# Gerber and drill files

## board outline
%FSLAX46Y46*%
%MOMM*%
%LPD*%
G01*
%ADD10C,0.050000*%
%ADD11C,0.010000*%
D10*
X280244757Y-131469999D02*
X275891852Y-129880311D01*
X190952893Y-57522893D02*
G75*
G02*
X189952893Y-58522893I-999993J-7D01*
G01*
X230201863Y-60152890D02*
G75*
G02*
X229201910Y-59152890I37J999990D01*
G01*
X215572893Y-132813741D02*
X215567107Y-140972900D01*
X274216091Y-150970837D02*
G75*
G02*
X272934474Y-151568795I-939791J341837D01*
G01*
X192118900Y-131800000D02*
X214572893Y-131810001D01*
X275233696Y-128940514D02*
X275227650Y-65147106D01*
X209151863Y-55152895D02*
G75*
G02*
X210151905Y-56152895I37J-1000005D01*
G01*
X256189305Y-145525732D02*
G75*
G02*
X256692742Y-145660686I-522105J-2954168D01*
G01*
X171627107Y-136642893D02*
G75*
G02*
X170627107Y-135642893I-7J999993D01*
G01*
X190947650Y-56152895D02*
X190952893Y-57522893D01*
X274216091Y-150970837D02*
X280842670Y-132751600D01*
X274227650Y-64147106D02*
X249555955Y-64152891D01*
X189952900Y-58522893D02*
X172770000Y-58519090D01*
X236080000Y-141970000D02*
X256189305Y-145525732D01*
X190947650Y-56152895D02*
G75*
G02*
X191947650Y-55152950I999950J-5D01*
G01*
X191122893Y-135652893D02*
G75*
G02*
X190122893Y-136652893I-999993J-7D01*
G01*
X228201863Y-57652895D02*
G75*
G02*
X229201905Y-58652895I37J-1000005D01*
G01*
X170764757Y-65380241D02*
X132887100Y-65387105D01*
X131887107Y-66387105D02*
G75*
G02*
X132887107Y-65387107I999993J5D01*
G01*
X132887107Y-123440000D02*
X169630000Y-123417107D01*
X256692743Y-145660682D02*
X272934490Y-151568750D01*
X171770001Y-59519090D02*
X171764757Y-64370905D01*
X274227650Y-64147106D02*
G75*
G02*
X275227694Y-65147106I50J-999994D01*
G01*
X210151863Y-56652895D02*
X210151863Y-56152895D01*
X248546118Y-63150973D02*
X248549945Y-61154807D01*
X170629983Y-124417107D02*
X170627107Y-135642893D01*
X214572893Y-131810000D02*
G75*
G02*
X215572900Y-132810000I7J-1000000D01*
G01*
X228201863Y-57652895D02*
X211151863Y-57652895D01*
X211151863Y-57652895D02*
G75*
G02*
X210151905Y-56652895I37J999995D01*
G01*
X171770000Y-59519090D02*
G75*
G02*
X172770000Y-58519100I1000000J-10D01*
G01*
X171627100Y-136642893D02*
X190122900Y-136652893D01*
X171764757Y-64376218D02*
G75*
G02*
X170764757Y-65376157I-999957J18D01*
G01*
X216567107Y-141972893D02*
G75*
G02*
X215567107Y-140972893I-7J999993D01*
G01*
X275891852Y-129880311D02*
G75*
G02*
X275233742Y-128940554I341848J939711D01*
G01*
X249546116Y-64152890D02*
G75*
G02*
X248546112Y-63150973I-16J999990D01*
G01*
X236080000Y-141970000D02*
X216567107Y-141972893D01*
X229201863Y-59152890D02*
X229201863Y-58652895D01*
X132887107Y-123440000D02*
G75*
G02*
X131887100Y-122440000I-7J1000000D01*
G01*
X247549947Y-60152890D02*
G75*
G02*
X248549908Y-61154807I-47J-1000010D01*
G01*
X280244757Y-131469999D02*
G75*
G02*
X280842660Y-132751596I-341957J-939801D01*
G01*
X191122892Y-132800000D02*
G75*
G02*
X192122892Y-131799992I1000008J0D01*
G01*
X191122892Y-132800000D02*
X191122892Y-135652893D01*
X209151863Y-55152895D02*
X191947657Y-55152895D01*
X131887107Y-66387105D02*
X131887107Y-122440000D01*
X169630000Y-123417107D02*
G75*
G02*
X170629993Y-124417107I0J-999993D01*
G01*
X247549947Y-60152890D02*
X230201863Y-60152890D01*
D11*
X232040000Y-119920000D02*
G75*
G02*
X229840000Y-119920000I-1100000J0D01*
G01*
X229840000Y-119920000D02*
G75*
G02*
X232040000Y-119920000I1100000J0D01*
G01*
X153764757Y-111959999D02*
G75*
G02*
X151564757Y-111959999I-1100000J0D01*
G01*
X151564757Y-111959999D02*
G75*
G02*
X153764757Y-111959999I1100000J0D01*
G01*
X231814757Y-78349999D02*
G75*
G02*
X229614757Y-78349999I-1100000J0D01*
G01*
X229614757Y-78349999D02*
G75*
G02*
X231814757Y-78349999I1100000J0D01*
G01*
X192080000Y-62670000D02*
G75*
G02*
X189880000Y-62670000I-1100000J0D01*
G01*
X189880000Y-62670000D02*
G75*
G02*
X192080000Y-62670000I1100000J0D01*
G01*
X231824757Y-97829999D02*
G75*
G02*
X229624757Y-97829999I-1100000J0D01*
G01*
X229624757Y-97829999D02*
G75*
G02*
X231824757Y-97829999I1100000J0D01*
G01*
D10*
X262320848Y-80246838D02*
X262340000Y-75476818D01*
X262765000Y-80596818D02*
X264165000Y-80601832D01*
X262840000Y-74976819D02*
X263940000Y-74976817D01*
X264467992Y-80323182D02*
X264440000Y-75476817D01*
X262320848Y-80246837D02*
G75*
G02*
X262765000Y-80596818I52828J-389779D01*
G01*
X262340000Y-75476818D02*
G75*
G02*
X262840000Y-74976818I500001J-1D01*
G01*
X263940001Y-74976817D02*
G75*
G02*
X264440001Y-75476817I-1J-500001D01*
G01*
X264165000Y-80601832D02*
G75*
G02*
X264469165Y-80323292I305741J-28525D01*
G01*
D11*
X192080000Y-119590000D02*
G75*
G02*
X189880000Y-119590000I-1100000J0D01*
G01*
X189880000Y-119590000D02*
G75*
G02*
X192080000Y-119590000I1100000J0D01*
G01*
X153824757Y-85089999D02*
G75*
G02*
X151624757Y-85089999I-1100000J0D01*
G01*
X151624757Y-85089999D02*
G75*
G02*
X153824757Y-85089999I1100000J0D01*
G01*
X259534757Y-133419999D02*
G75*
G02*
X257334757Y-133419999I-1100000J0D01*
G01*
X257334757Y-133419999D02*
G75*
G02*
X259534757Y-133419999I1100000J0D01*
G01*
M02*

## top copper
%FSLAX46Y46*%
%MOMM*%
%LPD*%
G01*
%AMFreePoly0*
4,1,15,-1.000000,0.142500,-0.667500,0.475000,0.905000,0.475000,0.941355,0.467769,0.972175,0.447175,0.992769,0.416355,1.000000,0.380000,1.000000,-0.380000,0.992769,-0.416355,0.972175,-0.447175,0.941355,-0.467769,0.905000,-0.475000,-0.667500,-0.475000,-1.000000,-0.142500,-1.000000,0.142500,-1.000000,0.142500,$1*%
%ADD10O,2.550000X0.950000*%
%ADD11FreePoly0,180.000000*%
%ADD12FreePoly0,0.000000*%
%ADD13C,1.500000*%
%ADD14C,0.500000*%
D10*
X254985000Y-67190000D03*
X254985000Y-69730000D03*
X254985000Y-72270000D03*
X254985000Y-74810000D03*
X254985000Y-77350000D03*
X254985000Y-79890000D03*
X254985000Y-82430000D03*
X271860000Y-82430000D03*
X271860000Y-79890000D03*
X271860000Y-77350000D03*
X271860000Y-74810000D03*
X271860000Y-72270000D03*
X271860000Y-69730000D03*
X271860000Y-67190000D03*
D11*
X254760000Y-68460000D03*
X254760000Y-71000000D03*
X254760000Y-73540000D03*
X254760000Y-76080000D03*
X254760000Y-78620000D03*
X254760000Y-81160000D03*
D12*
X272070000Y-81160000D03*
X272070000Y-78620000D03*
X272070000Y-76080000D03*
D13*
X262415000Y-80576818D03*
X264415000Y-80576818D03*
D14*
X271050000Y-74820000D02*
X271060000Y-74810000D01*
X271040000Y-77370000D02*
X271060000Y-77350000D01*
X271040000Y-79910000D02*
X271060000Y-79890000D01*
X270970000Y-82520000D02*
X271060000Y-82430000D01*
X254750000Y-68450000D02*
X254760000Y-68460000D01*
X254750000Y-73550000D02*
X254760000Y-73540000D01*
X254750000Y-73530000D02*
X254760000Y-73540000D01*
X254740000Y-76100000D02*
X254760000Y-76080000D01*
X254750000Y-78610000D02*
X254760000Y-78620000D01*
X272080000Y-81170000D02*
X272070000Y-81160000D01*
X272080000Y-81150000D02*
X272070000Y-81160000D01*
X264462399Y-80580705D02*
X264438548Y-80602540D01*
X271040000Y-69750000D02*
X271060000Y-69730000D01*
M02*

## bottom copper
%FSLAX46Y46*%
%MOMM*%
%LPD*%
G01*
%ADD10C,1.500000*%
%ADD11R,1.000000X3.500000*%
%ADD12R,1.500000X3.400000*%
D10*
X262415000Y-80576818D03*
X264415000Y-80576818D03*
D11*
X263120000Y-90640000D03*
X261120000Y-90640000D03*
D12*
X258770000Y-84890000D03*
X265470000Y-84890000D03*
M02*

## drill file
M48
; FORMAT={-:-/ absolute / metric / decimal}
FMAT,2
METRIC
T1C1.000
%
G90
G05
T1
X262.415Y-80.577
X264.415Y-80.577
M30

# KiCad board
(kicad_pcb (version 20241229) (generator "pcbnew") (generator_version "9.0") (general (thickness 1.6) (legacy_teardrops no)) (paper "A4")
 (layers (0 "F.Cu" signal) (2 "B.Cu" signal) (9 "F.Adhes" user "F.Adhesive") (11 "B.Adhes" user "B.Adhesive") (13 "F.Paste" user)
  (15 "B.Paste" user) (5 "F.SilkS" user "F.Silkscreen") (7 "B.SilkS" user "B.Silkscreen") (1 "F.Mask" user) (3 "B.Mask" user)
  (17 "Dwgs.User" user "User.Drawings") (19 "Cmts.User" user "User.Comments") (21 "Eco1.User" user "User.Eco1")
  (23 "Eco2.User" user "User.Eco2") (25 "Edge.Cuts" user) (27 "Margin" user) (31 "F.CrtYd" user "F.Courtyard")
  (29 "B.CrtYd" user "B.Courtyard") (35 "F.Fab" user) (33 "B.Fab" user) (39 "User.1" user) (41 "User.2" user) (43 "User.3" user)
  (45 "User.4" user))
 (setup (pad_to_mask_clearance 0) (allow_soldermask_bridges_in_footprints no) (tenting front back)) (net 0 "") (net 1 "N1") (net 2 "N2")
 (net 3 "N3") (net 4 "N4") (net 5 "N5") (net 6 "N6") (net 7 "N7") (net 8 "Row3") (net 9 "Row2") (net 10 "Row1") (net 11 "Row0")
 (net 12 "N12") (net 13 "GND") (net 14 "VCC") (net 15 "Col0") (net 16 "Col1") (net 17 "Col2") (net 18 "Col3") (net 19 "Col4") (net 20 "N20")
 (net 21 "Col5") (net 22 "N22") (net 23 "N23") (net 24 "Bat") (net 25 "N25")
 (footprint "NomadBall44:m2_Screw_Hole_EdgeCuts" (layer "F.Cu") (at 230.94 119.92)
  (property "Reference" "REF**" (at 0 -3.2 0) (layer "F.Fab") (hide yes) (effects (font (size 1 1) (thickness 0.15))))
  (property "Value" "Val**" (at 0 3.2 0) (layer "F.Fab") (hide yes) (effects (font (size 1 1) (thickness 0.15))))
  (fp_circle (center 0 0) (end 1.1 0) (stroke (width 0.01) (type solid)) (fill no) (layer "Edge.Cuts")))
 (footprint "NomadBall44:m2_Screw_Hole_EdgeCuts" (layer "F.Cu") (at 152.664757 111.959999)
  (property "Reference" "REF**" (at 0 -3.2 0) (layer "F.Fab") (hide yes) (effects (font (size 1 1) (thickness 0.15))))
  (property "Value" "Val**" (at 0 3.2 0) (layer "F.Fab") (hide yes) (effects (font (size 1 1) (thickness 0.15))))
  (fp_circle (center 0 0) (end 1.1 0) (stroke (width 0.01) (type solid)) (fill no) (layer "Edge.Cuts")))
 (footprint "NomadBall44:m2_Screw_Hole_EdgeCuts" (layer "F.Cu") (at 230.714757 78.349999)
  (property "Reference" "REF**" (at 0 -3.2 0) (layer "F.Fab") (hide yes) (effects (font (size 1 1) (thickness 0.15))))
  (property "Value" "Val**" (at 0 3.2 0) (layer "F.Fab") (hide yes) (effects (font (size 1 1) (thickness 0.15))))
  (fp_circle (center 0 0) (end 1.1 0) (stroke (width 0.01) (type solid)) (fill no) (layer "Edge.Cuts")))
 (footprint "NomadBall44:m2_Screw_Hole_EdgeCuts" (layer "F.Cu") (at 190.98 62.67)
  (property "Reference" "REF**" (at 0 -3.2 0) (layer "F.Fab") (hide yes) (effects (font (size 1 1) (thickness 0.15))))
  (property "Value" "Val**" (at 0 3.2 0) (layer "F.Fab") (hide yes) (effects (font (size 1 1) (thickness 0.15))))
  (fp_circle (center 0 0) (end 1.1 0) (stroke (width 0.01) (type solid)) (fill no) (layer "Edge.Cuts")))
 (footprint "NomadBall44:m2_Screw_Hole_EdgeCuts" (layer "F.Cu") (at 230.724757 97.829999)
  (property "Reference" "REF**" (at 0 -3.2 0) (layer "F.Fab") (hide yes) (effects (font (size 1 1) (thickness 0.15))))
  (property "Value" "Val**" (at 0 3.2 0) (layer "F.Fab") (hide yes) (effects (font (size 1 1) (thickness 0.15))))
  (fp_circle (center 0 0) (end 1.1 0) (stroke (width 0.01) (type solid)) (fill no) (layer "Edge.Cuts")))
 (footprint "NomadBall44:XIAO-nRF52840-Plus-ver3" (layer "F.Cu") (at 262.015 74.71 90)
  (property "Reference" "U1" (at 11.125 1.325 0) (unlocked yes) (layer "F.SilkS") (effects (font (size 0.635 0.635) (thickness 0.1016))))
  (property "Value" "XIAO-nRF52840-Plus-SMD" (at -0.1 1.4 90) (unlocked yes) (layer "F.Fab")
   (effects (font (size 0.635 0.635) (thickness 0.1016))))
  (fp_line (start -5.536838 0.305848) (end -0.766818 0.325) (stroke (width 0.05) (type default)) (layer "Edge.Cuts"))
  (fp_line (start -5.886818 0.75) (end -5.891832 2.15) (stroke (width 0.05) (type default)) (layer "Edge.Cuts"))
  (fp_line (start -0.266819 0.825) (end -0.266817 1.925) (stroke (width 0.05) (type default)) (layer "Edge.Cuts"))
  (fp_line (start -5.613182 2.452992) (end -0.766817 2.425) (stroke (width 0.05) (type default)) (layer "Edge.Cuts"))
  (fp_arc (start -5.536837 0.305848) (mid -5.617663 0.602123) (end -5.886818 0.75) (stroke (width 0.05) (type default)) (layer "Edge.Cuts"))
  (fp_arc (start -0.766818 0.325) (mid -0.413265 0.471447) (end -0.266818 0.825) (stroke (width 0.05) (type default)) (layer "Edge.Cuts"))
  (fp_arc (start -0.266817 1.925001) (mid -0.413264 2.278554) (end -0.766817 2.425001) (stroke (width 0.05) (type default))
   (layer "Edge.Cuts"))
  (fp_arc (start -5.891832 2.15) (mid -5.693897 2.24836) (end -5.613293 2.454165) (stroke (width 0.05) (type default)) (layer "Edge.Cuts"))
  (pad "1" smd oval (at 7.52 -6.23) (size 2.55 0.95) (drill (offset -0.8 0)) (layers "F.Cu" "F.Mask" "F.Paste") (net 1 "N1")
   (thermal_bridge_angle 45))
  (pad "2" smd oval (at 4.98 -6.23) (size 2.55 0.95) (drill (offset -0.8 0)) (layers "F.Cu" "F.Mask" "F.Paste") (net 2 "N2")
   (thermal_bridge_angle 45))
  (pad "3" smd oval (at 2.44 -6.23) (size 2.55 0.95) (drill (offset -0.8 0)) (layers "F.Cu" "F.Mask" "F.Paste") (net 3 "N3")
   (thermal_bridge_angle 45))
  (pad "4" smd oval (at -0.1 -6.23) (size 2.55 0.95) (drill (offset -0.8 0)) (layers "F.Cu" "F.Mask" "F.Paste") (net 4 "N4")
   (thermal_bridge_angle 45))
  (pad "5" smd oval (at -2.64 -6.23) (size 2.55 0.95) (drill (offset -0.8 0)) (layers "F.Cu" "F.Mask" "F.Paste") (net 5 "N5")
   (thermal_bridge_angle 45))
  (pad "6" smd oval (at -5.18 -6.23) (size 2.55 0.95) (drill (offset -0.8 0)) (layers "F.Cu" "F.Mask" "F.Paste") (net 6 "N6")
   (thermal_bridge_angle 45))
  (pad "7" smd oval (at -7.72 -6.23) (size 2.55 0.95) (drill (offset -0.8 0)) (layers "F.Cu" "F.Mask" "F.Paste") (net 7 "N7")
   (thermal_bridge_angle 45))
  (pad "8" smd oval (at -7.72 9.045) (size 2.55 0.95) (drill (offset 0.8 0)) (layers "F.Cu" "F.Mask" "F.Paste") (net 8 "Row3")
   (thermal_bridge_angle 45))
  (pad "9" smd oval (at -5.18 9.045) (size 2.55 0.95) (drill (offset 0.8 0)) (layers "F.Cu" "F.Mask" "F.Paste") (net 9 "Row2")
   (thermal_bridge_angle 45))
  (pad "10" smd oval (at -2.64 9.045) (size 2.55 0.95) (drill (offset 0.8 0)) (layers "F.Cu" "F.Mask" "F.Paste") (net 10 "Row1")
   (thermal_bridge_angle 45))
  (pad "11" smd oval (at -0.1 9.045) (size 2.55 0.95) (drill (offset 0.8 0)) (layers "F.Cu" "F.Mask" "F.Paste") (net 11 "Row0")
   (thermal_bridge_angle 45))
  (pad "12" smd oval (at 2.44 9.045) (size 2.55 0.95) (drill (offset 0.8 0)) (layers "F.Cu" "F.Mask" "F.Paste") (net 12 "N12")
   (thermal_bridge_angle 45))
  (pad "13" smd oval (at 4.98 9.045) (size 2.55 0.95) (drill (offset 0.8 0)) (layers "F.Cu" "F.Mask" "F.Paste") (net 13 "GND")
   (thermal_bridge_angle 45))
  (pad "14" smd oval (at 7.52 9.045) (size 2.55 0.95) (drill (offset 0.8 0)) (layers "F.Cu" "F.Mask" "F.Paste") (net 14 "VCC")
   (thermal_bridge_angle 45))
  (pad "15" smd roundrect (at 6.25 -7.255 180) (size 2 0.95) (layers "F.Cu" "F.Mask" "F.Paste") (roundrect_rratio 0.1) (chamfer_ratio 0.35)
   (chamfer top_left bottom_left) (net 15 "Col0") (thermal_bridge_angle 45))
  (pad "16" smd roundrect (at 3.71 -7.255 180) (size 2 0.95) (layers "F.Cu" "F.Mask" "F.Paste") (roundrect_rratio 0.1) (chamfer_ratio 0.35)
   (chamfer top_left bottom_left) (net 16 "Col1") (thermal_bridge_angle 45))
  (pad "17" smd roundrect (at 1.17 -7.255 180) (size 2 0.95) (layers "F.Cu" "F.Mask" "F.Paste") (roundrect_rratio 0.1) (chamfer_ratio 0.35)
   (chamfer top_left bottom_left) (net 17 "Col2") (thermal_bridge_angle 45))
  (pad "18" smd roundrect (at -1.37 -7.255 180) (size 2 0.95) (layers "F.Cu" "F.Mask" "F.Paste") (roundrect_rratio 0.1) (chamfer_ratio 0.35)
   (chamfer top_left bottom_left) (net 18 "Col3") (thermal_bridge_angle 45))
  (pad "19" smd roundrect (at -3.91 -7.255 180) (size 2 0.95) (layers "F.Cu" "F.Mask" "F.Paste") (roundrect_rratio 0.1) (chamfer_ratio 0.35)
   (chamfer top_left bottom_left) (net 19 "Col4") (thermal_bridge_angle 45))
  (pad "20" smd roundrect (at -6.45 -7.255 180) (size 2 0.95) (layers "F.Cu" "F.Mask" "F.Paste") (roundrect_rratio 0.1) (chamfer_ratio 0.35)
   (chamfer top_left bottom_left) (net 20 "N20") (thermal_bridge_angle 45))
  (pad "21" smd roundrect (at -6.45 10.055) (size 2 0.95) (layers "F.Cu" "F.Mask" "F.Paste") (roundrect_rratio 0.1) (chamfer_ratio 0.35)
   (chamfer top_left bottom_left) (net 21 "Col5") (thermal_bridge_angle 45))
  (pad "22" smd roundrect (at -3.91 10.055) (size 2 0.95) (layers "F.Cu" "F.Mask" "F.Paste") (roundrect_rratio 0.1) (chamfer_ratio 0.35)
   (chamfer top_left bottom_left) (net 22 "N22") (thermal_bridge_angle 45))
  (pad "23" smd roundrect (at -1.37 10.055) (size 2 0.95) (layers "F.Cu" "F.Mask" "F.Paste") (roundrect_rratio 0.1) (chamfer_ratio 0.35)
   (chamfer top_left bottom_left) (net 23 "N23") (thermal_bridge_angle 45))
  (pad "32" thru_hole circle (at -5.866818 0.4 90) (size 1.5 1.5) (drill 1) (layers "*.Cu" "*.Mask") (remove_unused_layers no)
   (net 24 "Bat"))
  (pad "33" thru_hole circle (at -5.866818 2.4 90) (size 1.5 1.5) (drill 1) (layers "*.Cu" "*.Mask") (remove_unused_layers no)
   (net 13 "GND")))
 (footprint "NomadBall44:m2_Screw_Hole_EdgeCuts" (layer "F.Cu") (at 190.98 119.59)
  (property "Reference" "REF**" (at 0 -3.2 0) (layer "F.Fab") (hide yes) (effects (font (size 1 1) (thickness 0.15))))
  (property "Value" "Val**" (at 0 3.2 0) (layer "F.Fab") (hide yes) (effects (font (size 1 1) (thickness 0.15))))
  (fp_circle (center 0 0) (end 1.1 0) (stroke (width 0.01) (type solid)) (fill no) (layer "Edge.Cuts")))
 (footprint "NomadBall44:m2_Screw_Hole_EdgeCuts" (layer "F.Cu") (at 152.724757 85.089999)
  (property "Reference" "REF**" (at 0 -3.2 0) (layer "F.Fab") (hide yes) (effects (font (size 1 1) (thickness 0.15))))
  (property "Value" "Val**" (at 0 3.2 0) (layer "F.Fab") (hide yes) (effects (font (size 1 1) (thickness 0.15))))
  (fp_circle (center 0 0) (end 1.1 0) (stroke (width 0.01) (type solid)) (fill no) (layer "Edge.Cuts")))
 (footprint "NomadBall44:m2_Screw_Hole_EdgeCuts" (layer "F.Cu") (at 258.434757 133.419999)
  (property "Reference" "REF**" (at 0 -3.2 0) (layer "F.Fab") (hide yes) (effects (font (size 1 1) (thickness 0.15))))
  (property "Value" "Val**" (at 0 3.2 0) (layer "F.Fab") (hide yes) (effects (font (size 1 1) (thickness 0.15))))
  (fp_circle (center 0 0) (end 1.1 0) (stroke (width 0.01) (type solid)) (fill no) (layer "Edge.Cuts")))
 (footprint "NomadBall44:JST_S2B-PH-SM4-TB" (layer "B.Cu") (at 262.12 90.64 180)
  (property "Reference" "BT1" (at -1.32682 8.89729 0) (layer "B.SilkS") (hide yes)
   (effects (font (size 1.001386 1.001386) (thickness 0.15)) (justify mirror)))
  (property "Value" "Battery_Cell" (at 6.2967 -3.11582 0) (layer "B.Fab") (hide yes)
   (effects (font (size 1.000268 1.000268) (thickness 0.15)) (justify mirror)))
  (pad "1" smd rect (at -1 0 180) (size 1 3.5) (layers "B.Cu" "B.Mask" "B.Paste") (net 24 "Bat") (solder_mask_margin 0.102))
  (pad "2" smd rect (at 1 0 180) (size 1 3.5) (layers "B.Cu" "B.Mask" "B.Paste") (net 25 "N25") (solder_mask_margin 0.102))
  (pad "P1" smd rect (at 3.35 5.75 180) (size 1.5 3.4) (layers "B.Cu" "B.Mask" "B.Paste") (solder_mask_margin 0.102))
  (pad "P2" smd rect (at -3.35 5.75 180) (size 1.5 3.4) (layers "B.Cu" "B.Mask" "B.Paste") (solder_mask_margin 0.102)))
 (gr_line (start 280.244757 131.469999) (end 275.891852 129.880311) (stroke (width 0.05) (type solid)) (layer "Edge.Cuts"))
 (gr_arc (start 190.952893 57.522893) (mid 190.66 58.23) (end 189.952893 58.522893) (stroke (width 0.05) (type solid)) (layer "Edge.Cuts"))
 (gr_arc (start 230.201863 60.15289) (mid 229.494756 59.859997) (end 229.201863 59.15289) (stroke (width 0.05) (type solid))
  (layer "Edge.Cuts"))
 (gr_line (start 215.572893 132.813741) (end 215.567107 140.9729) (stroke (width 0.05) (type default)) (layer "Edge.Cuts"))
 (gr_arc (start 274.216091 150.970837) (mid 273.699122 151.535222) (end 272.93449 151.56875) (stroke (width 0.05) (type solid))
  (layer "Edge.Cuts"))
 (gr_line (start 192.1189 131.8) (end 214.572893 131.810001) (stroke (width 0.05) (type default)) (layer "Edge.Cuts"))
 (gr_line (start 275.233696 128.940514) (end 275.22765 65.147106) (stroke (width 0.05) (type solid)) (layer "Edge.Cuts"))
 (gr_arc (start 209.151863 55.152895) (mid 209.85897 55.445788) (end 210.151863 56.152895) (stroke (width 0.05) (type solid))
  (layer "Edge.Cuts"))
 (gr_arc (start 256.189305 145.525732) (mid 256.443961 145.582253) (end 256.692744 145.660682) (stroke (width 0.05) (type solid))
  (layer "Edge.Cuts"))
 (gr_arc (start 171.627107 136.642893) (mid 170.92 136.35) (end 170.627107 135.642893) (stroke (width 0.05) (type solid))
  (layer "Edge.Cuts"))
 (gr_line (start 190.94765 56.152895) (end 190.952893 57.522893) (stroke (width 0.05) (type solid)) (layer "Edge.Cuts"))
 (gr_line (start 274.216091 150.970837) (end 280.84267 132.7516) (stroke (width 0.05) (type solid)) (layer "Edge.Cuts"))
 (gr_line (start 274.22765 64.147106) (end 249.555955 64.152891) (stroke (width 0.05) (type solid)) (layer "Edge.Cuts"))
 (gr_line (start 189.9529 58.522893) (end 172.77 58.51909) (stroke (width 0.05) (type solid)) (layer "Edge.Cuts"))
 (gr_line (start 236.08 141.97) (end 256.189305 145.525732) (stroke (width 0.05) (type solid)) (layer "Edge.Cuts"))
 (gr_arc (start 190.94765 56.152895) (mid 191.240543 55.445788) (end 191.94765 55.152895) (stroke (width 0.05) (type solid))
  (layer "Edge.Cuts"))
 (gr_arc (start 191.122893 135.652893) (mid 190.83 136.36) (end 190.122893 136.652893) (stroke (width 0.05) (type solid))
  (layer "Edge.Cuts"))
 (gr_arc (start 228.201863 57.652895) (mid 228.90897 57.945788) (end 229.201863 58.652895) (stroke (width 0.05) (type solid))
  (layer "Edge.Cuts"))
 (gr_line (start 170.764757 65.380241) (end 132.8871 65.387105) (stroke (width 0.05) (type solid)) (layer "Edge.Cuts"))
 (gr_arc (start 131.887107 66.387105) (mid 132.18 65.679998) (end 132.887107 65.387105) (stroke (width 0.05) (type solid))
  (layer "Edge.Cuts"))
 (gr_line (start 132.887107 123.44) (end 169.63 123.417107) (stroke (width 0.05) (type solid)) (layer "Edge.Cuts"))
 (gr_line (start 256.692743 145.660682) (end 272.93449 151.56875) (stroke (width 0.05) (type solid)) (layer "Edge.Cuts"))
 (gr_line (start 171.770001 59.51909) (end 171.764757 64.370905) (stroke (width 0.05) (type solid)) (layer "Edge.Cuts"))
 (gr_arc (start 274.22765 64.147106) (mid 274.934757 64.439999) (end 275.22765 65.147106) (stroke (width 0.05) (type solid))
  (layer "Edge.Cuts"))
 (gr_line (start 210.151863 56.652895) (end 210.151863 56.152895) (stroke (width 0.05) (type solid)) (layer "Edge.Cuts"))
 (gr_line (start 248.546118 63.150973) (end 248.549945 61.154807) (stroke (width 0.05) (type solid)) (layer "Edge.Cuts"))
 (gr_line (start 170.629983 124.417107) (end 170.627107 135.642893) (stroke (width 0.05) (type default)) (layer "Edge.Cuts"))
 (gr_arc (start 214.572893 131.81) (mid 215.28 132.102893) (end 215.572893 132.81) (stroke (width 0.05) (type solid)) (layer "Edge.Cuts"))
 (gr_line (start 228.201863 57.652895) (end 211.151863 57.652895) (stroke (width 0.05) (type solid)) (layer "Edge.Cuts"))
 (gr_arc (start 211.151863 57.652895) (mid 210.444756 57.360002) (end 210.151863 56.652895) (stroke (width 0.05) (type solid))
  (layer "Edge.Cuts"))
 (gr_arc (start 171.77 59.51909) (mid 172.062893 58.811983) (end 172.77 58.51909) (stroke (width 0.05) (type solid)) (layer "Edge.Cuts"))
 (gr_line (start 171.6271 136.642893) (end 190.1229 136.652893) (stroke (width 0.05) (type solid)) (layer "Edge.Cuts"))
 (gr_arc (start 171.764757 64.376218) (mid 171.471864 65.083325) (end 170.764757 65.376218) (stroke (width 0.05) (type solid))
  (layer "Edge.Cuts"))
 (gr_arc (start 216.567107 141.972893) (mid 215.86 141.68) (end 215.567107 140.972893) (stroke (width 0.05) (type solid))
  (layer "Edge.Cuts"))
 (gr_arc (start 275.891852 129.880311) (mid 275.414594 129.51421) (end 275.233696 128.940554) (stroke (width 0.05) (type solid))
  (layer "Edge.Cuts"))
 (gr_arc (start 249.546116 64.15289) (mid 248.838332 63.859319) (end 248.546118 63.150973) (stroke (width 0.05) (type solid))
  (layer "Edge.Cuts"))
 (gr_line (start 236.08 141.97) (end 216.567107 141.972893) (stroke (width 0.05) (type default)) (layer "Edge.Cuts"))
 (gr_line (start 229.201863 59.15289) (end 229.201863 58.652895) (stroke (width 0.05) (type solid)) (layer "Edge.Cuts"))
 (gr_arc (start 132.887107 123.44) (mid 132.18 123.147107) (end 131.887107 122.44) (stroke (width 0.05) (type solid)) (layer "Edge.Cuts"))
 (gr_arc (start 247.549947 60.15289) (mid 248.257731 60.446461) (end 248.549945 61.154807) (stroke (width 0.05) (type solid))
  (layer "Edge.Cuts"))
 (gr_arc (start 280.244757 131.469999) (mid 280.809115 131.98698) (end 280.84267 132.7516) (stroke (width 0.05) (type solid))
  (layer "Edge.Cuts"))
 (gr_arc (start 191.122892 132.8) (mid 191.415785 132.092893) (end 192.122892 131.8) (stroke (width 0.05) (type solid)) (layer "Edge.Cuts"))
 (gr_line (start 191.122892 132.8) (end 191.122892 135.652893) (stroke (width 0.05) (type solid)) (layer "Edge.Cuts"))
 (gr_line (start 209.151863 55.152895) (end 191.947657 55.152895) (stroke (width 0.05) (type solid)) (layer "Edge.Cuts"))
 (gr_line (start 131.887107 66.387105) (end 131.887107 122.44) (stroke (width 0.05) (type solid)) (layer "Edge.Cuts"))
 (gr_arc (start 169.63 123.417107) (mid 170.337107 123.71) (end 170.63 124.417107) (stroke (width 0.05) (type solid)) (layer "Edge.Cuts"))
 (gr_line (start 247.549947 60.15289) (end 230.201863 60.15289) (stroke (width 0.05) (type solid)) (layer "Edge.Cuts"))
 (segment (start 271.05 74.82) (end 271.06 74.81) (width 0.5) (layer "F.Cu") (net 11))
 (segment (start 271.04 77.37) (end 271.06 77.35) (width 0.5) (layer "F.Cu") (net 10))
 (segment (start 271.04 79.91) (end 271.06 79.89) (width 0.5) (layer "F.Cu") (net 9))
 (segment (start 270.97 82.52) (end 271.06 82.43) (width 0.5) (layer "F.Cu") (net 8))
 (segment (start 254.75 68.45) (end 254.76 68.46) (width 0.5) (layer "F.Cu") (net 15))
 (segment (start 254.75 73.55) (end 254.76 73.54) (width 0.5) (layer "F.Cu") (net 17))
 (segment (start 254.75 73.53) (end 254.76 73.54) (width 0.5) (layer "F.Cu") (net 17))
 (segment (start 254.74 76.1) (end 254.76 76.08) (width 0.5) (layer "F.Cu") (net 18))
 (segment (start 254.75 78.61) (end 254.76 78.62) (width 0.5) (layer "F.Cu") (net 19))
 (segment (start 272.08 81.17) (end 272.07 81.16) (width 0.5) (layer "F.Cu") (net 21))
 (segment (start 272.08 81.15) (end 272.07 81.16) (width 0.5) (layer "F.Cu") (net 21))
 (segment (start 264.462399 80.580705) (end 264.438548 80.60254) (width 0.5) (layer "F.Cu") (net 13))
 (segment (start 271.04 69.75) (end 271.06 69.73) (width 0.5) (layer "F.Cu") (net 13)))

